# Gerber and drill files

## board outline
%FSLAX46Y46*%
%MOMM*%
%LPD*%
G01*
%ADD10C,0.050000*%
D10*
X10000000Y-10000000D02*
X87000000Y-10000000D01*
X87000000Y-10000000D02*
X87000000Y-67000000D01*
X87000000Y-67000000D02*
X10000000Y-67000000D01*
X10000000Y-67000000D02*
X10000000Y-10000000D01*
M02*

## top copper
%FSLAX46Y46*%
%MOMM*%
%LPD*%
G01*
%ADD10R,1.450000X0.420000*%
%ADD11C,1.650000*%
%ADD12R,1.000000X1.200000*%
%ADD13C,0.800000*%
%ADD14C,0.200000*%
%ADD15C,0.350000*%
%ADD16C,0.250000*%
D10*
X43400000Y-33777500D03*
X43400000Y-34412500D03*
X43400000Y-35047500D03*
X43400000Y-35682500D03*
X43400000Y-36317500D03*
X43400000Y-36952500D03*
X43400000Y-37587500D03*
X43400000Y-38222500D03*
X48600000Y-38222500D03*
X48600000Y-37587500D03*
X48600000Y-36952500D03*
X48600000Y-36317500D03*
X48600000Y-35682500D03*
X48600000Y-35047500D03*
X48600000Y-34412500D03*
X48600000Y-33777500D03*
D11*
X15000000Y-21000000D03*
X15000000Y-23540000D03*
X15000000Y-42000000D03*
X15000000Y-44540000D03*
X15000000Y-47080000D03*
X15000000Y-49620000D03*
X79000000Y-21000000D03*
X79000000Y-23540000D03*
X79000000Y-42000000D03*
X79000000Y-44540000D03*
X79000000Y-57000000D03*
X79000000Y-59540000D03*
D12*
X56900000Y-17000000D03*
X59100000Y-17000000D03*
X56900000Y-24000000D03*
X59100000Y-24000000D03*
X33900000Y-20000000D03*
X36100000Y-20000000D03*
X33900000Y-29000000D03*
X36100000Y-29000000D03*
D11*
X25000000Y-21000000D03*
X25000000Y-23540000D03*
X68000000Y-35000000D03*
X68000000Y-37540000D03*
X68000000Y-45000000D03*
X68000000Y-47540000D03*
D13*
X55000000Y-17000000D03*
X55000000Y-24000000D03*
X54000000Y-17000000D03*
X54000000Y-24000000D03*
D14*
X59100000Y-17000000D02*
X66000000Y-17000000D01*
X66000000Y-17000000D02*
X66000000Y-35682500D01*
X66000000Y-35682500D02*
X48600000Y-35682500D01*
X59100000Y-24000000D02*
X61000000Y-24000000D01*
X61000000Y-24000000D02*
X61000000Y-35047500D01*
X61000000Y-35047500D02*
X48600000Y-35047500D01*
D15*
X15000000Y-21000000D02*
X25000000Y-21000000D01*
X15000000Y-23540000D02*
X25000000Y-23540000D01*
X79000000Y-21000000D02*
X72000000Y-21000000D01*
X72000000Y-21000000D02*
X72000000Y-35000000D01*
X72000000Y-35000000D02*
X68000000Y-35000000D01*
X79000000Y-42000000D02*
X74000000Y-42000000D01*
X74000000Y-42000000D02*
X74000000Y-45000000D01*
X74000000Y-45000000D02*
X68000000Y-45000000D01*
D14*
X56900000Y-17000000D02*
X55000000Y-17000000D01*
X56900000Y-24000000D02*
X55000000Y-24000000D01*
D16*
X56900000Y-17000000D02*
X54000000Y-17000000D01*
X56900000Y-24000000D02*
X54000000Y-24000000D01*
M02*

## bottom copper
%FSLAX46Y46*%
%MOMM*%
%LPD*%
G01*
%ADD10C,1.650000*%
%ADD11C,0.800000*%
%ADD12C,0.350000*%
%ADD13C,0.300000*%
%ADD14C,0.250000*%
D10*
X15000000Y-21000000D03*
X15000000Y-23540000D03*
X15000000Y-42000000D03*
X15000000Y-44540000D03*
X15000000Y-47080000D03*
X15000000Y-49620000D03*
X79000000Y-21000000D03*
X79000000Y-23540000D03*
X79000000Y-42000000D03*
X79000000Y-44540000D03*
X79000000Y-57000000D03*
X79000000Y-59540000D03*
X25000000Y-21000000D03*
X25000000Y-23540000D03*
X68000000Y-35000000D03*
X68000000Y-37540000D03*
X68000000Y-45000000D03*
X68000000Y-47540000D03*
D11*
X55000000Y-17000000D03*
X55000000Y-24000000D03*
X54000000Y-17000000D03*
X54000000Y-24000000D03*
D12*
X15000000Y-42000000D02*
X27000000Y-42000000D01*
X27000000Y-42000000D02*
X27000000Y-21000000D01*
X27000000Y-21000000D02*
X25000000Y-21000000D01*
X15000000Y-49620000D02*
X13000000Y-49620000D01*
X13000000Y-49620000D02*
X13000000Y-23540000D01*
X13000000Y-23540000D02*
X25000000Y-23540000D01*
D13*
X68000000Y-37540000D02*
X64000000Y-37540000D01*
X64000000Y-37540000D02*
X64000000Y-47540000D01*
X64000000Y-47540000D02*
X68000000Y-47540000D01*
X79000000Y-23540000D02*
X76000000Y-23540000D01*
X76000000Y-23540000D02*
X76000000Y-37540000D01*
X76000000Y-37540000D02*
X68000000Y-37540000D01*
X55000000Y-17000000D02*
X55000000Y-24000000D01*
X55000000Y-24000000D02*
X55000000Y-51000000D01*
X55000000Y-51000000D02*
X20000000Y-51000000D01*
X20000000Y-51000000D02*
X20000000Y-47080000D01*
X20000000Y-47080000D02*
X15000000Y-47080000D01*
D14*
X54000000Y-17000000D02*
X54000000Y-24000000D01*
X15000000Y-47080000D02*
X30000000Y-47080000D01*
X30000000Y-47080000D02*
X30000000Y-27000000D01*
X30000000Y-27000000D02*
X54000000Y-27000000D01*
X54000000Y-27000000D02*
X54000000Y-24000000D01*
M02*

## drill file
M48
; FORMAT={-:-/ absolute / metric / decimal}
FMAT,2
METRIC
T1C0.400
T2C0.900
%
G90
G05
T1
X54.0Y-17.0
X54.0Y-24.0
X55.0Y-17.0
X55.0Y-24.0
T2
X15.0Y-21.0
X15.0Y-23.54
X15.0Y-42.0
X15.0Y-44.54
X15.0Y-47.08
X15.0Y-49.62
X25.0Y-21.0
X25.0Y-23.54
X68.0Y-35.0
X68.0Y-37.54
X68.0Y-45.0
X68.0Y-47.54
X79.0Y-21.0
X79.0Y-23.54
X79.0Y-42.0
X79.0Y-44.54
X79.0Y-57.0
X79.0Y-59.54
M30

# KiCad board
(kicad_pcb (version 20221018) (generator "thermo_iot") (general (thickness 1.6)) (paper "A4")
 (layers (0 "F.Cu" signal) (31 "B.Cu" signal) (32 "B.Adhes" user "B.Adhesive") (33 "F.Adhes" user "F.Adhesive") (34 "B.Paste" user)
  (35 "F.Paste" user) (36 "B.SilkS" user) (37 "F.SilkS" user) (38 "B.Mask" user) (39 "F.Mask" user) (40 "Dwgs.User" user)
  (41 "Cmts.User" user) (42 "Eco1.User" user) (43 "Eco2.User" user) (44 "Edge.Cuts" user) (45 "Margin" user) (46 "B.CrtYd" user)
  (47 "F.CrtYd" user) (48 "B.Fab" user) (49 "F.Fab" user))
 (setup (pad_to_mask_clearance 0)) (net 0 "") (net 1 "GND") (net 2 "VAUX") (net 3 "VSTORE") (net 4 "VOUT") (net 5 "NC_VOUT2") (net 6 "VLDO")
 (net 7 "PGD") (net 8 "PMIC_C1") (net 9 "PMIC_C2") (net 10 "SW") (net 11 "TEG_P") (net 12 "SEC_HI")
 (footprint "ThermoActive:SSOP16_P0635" (layer "F.Cu") (at 46 36)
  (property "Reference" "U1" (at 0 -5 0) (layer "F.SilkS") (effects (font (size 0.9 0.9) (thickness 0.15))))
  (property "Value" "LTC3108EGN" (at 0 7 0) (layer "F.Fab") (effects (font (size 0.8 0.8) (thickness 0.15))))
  (pad "1" smd rect (at -2.6 -2.2225) (size 1.45 0.42) (layers "F.Cu" "F.Paste" "F.Mask") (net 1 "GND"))
  (pad "2" smd rect (at -2.6 -1.5875) (size 1.45 0.42) (layers "F.Cu" "F.Paste" "F.Mask") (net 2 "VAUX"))
  (pad "3" smd rect (at -2.6 -0.9525) (size 1.45 0.42) (layers "F.Cu" "F.Paste" "F.Mask") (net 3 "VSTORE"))
  (pad "4" smd rect (at -2.6 -0.3175) (size 1.45 0.42) (layers "F.Cu" "F.Paste" "F.Mask") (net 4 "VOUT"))
  (pad "5" smd rect (at -2.6 0.3175) (size 1.45 0.42) (layers "F.Cu" "F.Paste" "F.Mask") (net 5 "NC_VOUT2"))
  (pad "6" smd rect (at -2.6 0.9525) (size 1.45 0.42) (layers "F.Cu" "F.Paste" "F.Mask") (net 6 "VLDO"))
  (pad "7" smd rect (at -2.6 1.5875) (size 1.45 0.42) (layers "F.Cu" "F.Paste" "F.Mask") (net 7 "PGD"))
  (pad "8" smd rect (at -2.6 2.2225) (size 1.45 0.42) (layers "F.Cu" "F.Paste" "F.Mask") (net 1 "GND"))
  (pad "9" smd rect (at 2.6 2.2225) (size 1.45 0.42) (layers "F.Cu" "F.Paste" "F.Mask") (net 1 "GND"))
  (pad "10" smd rect (at 2.6 1.5875) (size 1.45 0.42) (layers "F.Cu" "F.Paste" "F.Mask") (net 1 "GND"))
  (pad "11" smd rect (at 2.6 0.9525) (size 1.45 0.42) (layers "F.Cu" "F.Paste" "F.Mask") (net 2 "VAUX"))
  (pad "12" smd rect (at 2.6 0.3175) (size 1.45 0.42) (layers "F.Cu" "F.Paste" "F.Mask") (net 1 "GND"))
  (pad "13" smd rect (at 2.6 -0.3175) (size 1.45 0.42) (layers "F.Cu" "F.Paste" "F.Mask") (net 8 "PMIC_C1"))
  (pad "14" smd rect (at 2.6 -0.9525) (size 1.45 0.42) (layers "F.Cu" "F.Paste" "F.Mask") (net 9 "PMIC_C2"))
  (pad "15" smd rect (at 2.6 -1.5875) (size 1.45 0.42) (layers "F.Cu" "F.Paste" "F.Mask") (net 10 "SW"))
  (pad "16" smd rect (at 2.6 -2.2225) (size 1.45 0.42) (layers "F.Cu" "F.Paste" "F.Mask") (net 1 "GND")))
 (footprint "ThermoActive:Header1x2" (layer "F.Cu") (at 15 21)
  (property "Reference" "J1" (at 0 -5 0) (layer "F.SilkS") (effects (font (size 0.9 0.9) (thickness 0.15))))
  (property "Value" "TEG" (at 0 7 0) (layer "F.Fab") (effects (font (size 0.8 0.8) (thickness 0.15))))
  (pad "1" thru_hole circle (at 0 0) (size 1.65 1.65) (drill 0.9) (layers "*.Cu" "*.Mask") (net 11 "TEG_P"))
  (pad "2" thru_hole circle (at 0 2.54) (size 1.65 1.65) (drill 0.9) (layers "*.Cu" "*.Mask") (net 1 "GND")))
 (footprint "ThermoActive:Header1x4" (layer "F.Cu") (at 15 42)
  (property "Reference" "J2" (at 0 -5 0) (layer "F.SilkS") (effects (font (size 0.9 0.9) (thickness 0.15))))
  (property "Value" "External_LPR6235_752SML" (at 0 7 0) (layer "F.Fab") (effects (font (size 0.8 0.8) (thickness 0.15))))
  (pad "1" thru_hole circle (at 0 0) (size 1.65 1.65) (drill 0.9) (layers "*.Cu" "*.Mask") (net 11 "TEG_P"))
  (pad "2" thru_hole circle (at 0 2.54) (size 1.65 1.65) (drill 0.9) (layers "*.Cu" "*.Mask") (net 10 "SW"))
  (pad "3" thru_hole circle (at 0 5.08) (size 1.65 1.65) (drill 0.9) (layers "*.Cu" "*.Mask") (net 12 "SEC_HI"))
  (pad "4" thru_hole circle (at 0 7.62) (size 1.65 1.65) (drill 0.9) (layers "*.Cu" "*.Mask") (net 1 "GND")))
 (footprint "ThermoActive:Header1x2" (layer "F.Cu") (at 79 21)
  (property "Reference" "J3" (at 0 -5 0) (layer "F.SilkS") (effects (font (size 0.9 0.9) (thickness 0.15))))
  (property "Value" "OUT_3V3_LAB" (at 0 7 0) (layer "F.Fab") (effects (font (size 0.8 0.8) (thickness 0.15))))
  (pad "1" thru_hole circle (at 0 0) (size 1.65 1.65) (drill 0.9) (layers "*.Cu" "*.Mask") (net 4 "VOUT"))
  (pad "2" thru_hole circle (at 0 2.54) (size 1.65 1.65) (drill 0.9) (layers "*.Cu" "*.Mask") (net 1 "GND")))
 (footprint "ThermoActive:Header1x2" (layer "F.Cu") (at 79 42)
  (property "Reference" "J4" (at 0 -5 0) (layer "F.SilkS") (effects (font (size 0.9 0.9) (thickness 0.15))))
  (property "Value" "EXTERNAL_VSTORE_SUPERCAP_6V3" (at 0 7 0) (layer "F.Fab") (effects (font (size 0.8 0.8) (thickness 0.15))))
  (pad "1" thru_hole circle (at 0 0) (size 1.65 1.65) (drill 0.9) (layers "*.Cu" "*.Mask") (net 3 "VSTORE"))
  (pad "2" thru_hole circle (at 0 2.54) (size 1.65 1.65) (drill 0.9) (layers "*.Cu" "*.Mask") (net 1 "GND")))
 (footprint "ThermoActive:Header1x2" (layer "F.Cu") (at 79 57)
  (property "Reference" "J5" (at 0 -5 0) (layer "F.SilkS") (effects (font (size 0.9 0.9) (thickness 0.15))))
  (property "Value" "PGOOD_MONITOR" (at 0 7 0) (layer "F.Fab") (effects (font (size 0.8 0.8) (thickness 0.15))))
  (pad "1" thru_hole circle (at 0 0) (size 1.65 1.65) (drill 0.9) (layers "*.Cu" "*.Mask") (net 7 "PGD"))
  (pad "2" thru_hole circle (at 0 2.54) (size 1.65 1.65) (drill 0.9) (layers "*.Cu" "*.Mask") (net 1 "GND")))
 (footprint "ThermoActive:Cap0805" (layer "F.Cu") (at 58 17)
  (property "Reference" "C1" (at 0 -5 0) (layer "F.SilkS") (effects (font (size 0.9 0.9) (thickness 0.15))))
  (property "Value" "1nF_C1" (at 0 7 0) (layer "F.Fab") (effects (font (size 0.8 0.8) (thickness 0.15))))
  (pad "1" smd rect (at -1.1 0) (size 1 1.2) (layers "F.Cu" "F.Paste" "F.Mask") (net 12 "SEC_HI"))
  (pad "2" smd rect (at 1.1 0) (size 1 1.2) (layers "F.Cu" "F.Paste" "F.Mask") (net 8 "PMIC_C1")))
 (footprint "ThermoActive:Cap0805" (layer "F.Cu") (at 58 24)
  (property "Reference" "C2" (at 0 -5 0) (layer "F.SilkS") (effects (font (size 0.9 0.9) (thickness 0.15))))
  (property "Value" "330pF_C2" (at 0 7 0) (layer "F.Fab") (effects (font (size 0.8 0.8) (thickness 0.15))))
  (pad "1" smd rect (at -1.1 0) (size 1 1.2) (layers "F.Cu" "F.Paste" "F.Mask") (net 12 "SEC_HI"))
  (pad "2" smd rect (at 1.1 0) (size 1 1.2) (layers "F.Cu" "F.Paste" "F.Mask") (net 9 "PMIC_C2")))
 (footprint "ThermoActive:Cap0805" (layer "F.Cu") (at 35 20)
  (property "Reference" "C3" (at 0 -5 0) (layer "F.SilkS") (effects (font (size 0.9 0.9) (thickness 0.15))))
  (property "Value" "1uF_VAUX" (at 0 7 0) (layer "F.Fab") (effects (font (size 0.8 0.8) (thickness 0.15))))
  (pad "1" smd rect (at -1.1 0) (size 1 1.2) (layers "F.Cu" "F.Paste" "F.Mask") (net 2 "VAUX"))
  (pad "2" smd rect (at 1.1 0) (size 1 1.2) (layers "F.Cu" "F.Paste" "F.Mask") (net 1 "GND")))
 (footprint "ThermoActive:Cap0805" (layer "F.Cu") (at 35 29)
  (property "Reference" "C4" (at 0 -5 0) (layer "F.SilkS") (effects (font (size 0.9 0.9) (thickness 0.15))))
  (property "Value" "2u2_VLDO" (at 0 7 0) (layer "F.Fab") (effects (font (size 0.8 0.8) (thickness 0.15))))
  (pad "1" smd rect (at -1.1 0) (size 1 1.2) (layers "F.Cu" "F.Paste" "F.Mask") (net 6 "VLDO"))
  (pad "2" smd rect (at 1.1 0) (size 1 1.2) (layers "F.Cu" "F.Paste" "F.Mask") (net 1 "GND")))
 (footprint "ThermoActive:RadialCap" (layer "F.Cu") (at 25 21)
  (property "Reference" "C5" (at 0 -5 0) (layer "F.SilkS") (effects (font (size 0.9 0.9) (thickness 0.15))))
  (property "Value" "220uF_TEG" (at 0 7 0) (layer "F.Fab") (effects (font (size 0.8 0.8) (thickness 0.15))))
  (pad "1" thru_hole circle (at 0 0) (size 1.65 1.65) (drill 0.9) (layers "*.Cu" "*.Mask") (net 11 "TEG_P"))
  (pad "2" thru_hole circle (at 0 2.54) (size 1.65 1.65) (drill 0.9) (layers "*.Cu" "*.Mask") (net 1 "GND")))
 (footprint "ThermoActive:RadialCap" (layer "F.Cu") (at 68 35)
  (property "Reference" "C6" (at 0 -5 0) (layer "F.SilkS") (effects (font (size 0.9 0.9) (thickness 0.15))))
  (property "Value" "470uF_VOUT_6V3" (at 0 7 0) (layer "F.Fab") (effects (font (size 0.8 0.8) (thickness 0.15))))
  (pad "1" thru_hole circle (at 0 0) (size 1.65 1.65) (drill 0.9) (layers "*.Cu" "*.Mask") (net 4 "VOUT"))
  (pad "2" thru_hole circle (at 0 2.54) (size 1.65 1.65) (drill 0.9) (layers "*.Cu" "*.Mask") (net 1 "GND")))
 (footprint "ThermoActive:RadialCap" (layer "F.Cu") (at 68 45)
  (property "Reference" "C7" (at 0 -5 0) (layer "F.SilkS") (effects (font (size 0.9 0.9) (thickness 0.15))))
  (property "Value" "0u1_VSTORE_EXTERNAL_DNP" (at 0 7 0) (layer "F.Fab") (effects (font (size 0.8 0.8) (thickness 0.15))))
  (pad "1" thru_hole circle (at 0 0) (size 1.65 1.65) (drill 0.9) (layers "*.Cu" "*.Mask") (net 3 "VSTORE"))
  (pad "2" thru_hole circle (at 0 2.54) (size 1.65 1.65) (drill 0.9) (layers "*.Cu" "*.Mask") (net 1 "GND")))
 (segment (start 59.1 17) (end 66 17) (width 0.2) (layer "F.Cu") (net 8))
 (segment (start 66 17) (end 66 35.6825) (width 0.2) (layer "F.Cu") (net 8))
 (segment (start 66 35.6825) (end 48.6 35.6825) (width 0.2) (layer "F.Cu") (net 8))
 (segment (start 59.1 24) (end 61 24) (width 0.2) (layer "F.Cu") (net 9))
 (segment (start 61 24) (end 61 35.0475) (width 0.2) (layer "F.Cu") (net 9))
 (segment (start 61 35.0475) (end 48.6 35.0475) (width 0.2) (layer "F.Cu") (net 9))
 (segment (start 15 21) (end 25 21) (width 0.35) (layer "F.Cu") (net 11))
 (segment (start 15 23.54) (end 25 23.54) (width 0.35) (layer "F.Cu") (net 1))
 (segment (start 15 42) (end 27 42) (width 0.35) (layer "B.Cu") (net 11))
 (segment (start 27 42) (end 27 21) (width 0.35) (layer "B.Cu") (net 11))
 (segment (start 27 21) (end 25 21) (width 0.35) (layer "B.Cu") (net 11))
 (segment (start 15 49.62) (end 13 49.62) (width 0.35) (layer "B.Cu") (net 1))
 (segment (start 13 49.62) (end 13 23.54) (width 0.35) (layer "B.Cu") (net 1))
 (segment (start 13 23.54) (end 25 23.54) (width 0.35) (layer "B.Cu") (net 1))
 (segment (start 79 21) (end 72 21) (width 0.35) (layer "F.Cu") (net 4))
 (segment (start 72 21) (end 72 35) (width 0.35) (layer "F.Cu") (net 4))
 (segment (start 72 35) (end 68 35) (width 0.35) (layer "F.Cu") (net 4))
 (segment (start 79 42) (end 74 42) (width 0.35) (layer "F.Cu") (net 3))
 (segment (start 74 42) (end 74 45) (width 0.35) (layer "F.Cu") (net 3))
 (segment (start 74 45) (end 68 45) (width 0.35) (layer "F.Cu") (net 3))
 (segment (start 68 37.54) (end 64 37.54) (width 0.3) (layer "B.Cu") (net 1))
 (segment (start 64 37.54) (end 64 47.54) (width 0.3) (layer "B.Cu") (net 1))
 (segment (start 64 47.54) (end 68 47.54) (width 0.3) (layer "B.Cu") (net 1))
 (segment (start 79 23.54) (end 76 23.54) (width 0.3) (layer "B.Cu") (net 1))
 (segment (start 76 23.54) (end 76 37.54) (width 0.3) (layer "B.Cu") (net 1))
 (segment (start 76 37.54) (end 68 37.54) (width 0.3) (layer "B.Cu") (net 1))
 (segment (start 56.9 17) (end 55 17) (width 0.2) (layer "F.Cu") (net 12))
 (segment (start 56.9 24) (end 55 24) (width 0.2) (layer "F.Cu") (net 12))
 (segment (start 55 17) (end 55 24) (width 0.3) (layer "B.Cu") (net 12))
 (segment (start 55 24) (end 55 51) (width 0.3) (layer "B.Cu") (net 12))
 (segment (start 55 51) (end 20 51) (width 0.3) (layer "B.Cu") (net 12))
 (segment (start 20 51) (end 20 47.08) (width 0.3) (layer "B.Cu") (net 12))
 (segment (start 20 47.08) (end 15 47.08) (width 0.3) (layer "B.Cu") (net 12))
 (via (at 55 17) (size 0.8) (drill 0.4) (layers "F.Cu" "B.Cu") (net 12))
 (via (at 55 24) (size 0.8) (drill 0.4) (layers "F.Cu" "B.Cu") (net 12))
 (segment (start 56.9 17) (end 54 17) (width 0.25) (layer "F.Cu") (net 12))
 (segment (start 56.9 24) (end 54 24) (width 0.25) (layer "F.Cu") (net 12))
 (segment (start 54 17) (end 54 24) (width 0.25) (layer "B.Cu") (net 12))
 (segment (start 15 47.08) (end 30 47.08) (width 0.25) (layer "B.Cu") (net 12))
 (segment (start 30 47.08) (end 30 27) (width 0.25) (layer "B.Cu") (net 12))
 (segment (start 30 27) (end 54 27) (width 0.25) (layer "B.Cu") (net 12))
 (segment (start 54 27) (end 54 24) (width 0.25) (layer "B.Cu") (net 12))
 (via (at 54 17) (size 0.8) (drill 0.4) (layers "F.Cu" "B.Cu") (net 12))
 (via (at 54 24) (size 0.8) (drill 0.4) (layers "F.Cu" "B.Cu") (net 12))
 (gr_line (start 10 10) (end 87 10) (stroke (width 0.05) (type default)) (layer "Edge.Cuts"))
 (gr_line (start 87 10) (end 87 67) (stroke (width 0.05) (type default)) (layer "Edge.Cuts"))
 (gr_line (start 87 67) (end 10 67) (stroke (width 0.05) (type default)) (layer "Edge.Cuts"))
 (gr_line (start 10 67) (end 10 10) (stroke (width 0.05) (type default)) (layer "Edge.Cuts")))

